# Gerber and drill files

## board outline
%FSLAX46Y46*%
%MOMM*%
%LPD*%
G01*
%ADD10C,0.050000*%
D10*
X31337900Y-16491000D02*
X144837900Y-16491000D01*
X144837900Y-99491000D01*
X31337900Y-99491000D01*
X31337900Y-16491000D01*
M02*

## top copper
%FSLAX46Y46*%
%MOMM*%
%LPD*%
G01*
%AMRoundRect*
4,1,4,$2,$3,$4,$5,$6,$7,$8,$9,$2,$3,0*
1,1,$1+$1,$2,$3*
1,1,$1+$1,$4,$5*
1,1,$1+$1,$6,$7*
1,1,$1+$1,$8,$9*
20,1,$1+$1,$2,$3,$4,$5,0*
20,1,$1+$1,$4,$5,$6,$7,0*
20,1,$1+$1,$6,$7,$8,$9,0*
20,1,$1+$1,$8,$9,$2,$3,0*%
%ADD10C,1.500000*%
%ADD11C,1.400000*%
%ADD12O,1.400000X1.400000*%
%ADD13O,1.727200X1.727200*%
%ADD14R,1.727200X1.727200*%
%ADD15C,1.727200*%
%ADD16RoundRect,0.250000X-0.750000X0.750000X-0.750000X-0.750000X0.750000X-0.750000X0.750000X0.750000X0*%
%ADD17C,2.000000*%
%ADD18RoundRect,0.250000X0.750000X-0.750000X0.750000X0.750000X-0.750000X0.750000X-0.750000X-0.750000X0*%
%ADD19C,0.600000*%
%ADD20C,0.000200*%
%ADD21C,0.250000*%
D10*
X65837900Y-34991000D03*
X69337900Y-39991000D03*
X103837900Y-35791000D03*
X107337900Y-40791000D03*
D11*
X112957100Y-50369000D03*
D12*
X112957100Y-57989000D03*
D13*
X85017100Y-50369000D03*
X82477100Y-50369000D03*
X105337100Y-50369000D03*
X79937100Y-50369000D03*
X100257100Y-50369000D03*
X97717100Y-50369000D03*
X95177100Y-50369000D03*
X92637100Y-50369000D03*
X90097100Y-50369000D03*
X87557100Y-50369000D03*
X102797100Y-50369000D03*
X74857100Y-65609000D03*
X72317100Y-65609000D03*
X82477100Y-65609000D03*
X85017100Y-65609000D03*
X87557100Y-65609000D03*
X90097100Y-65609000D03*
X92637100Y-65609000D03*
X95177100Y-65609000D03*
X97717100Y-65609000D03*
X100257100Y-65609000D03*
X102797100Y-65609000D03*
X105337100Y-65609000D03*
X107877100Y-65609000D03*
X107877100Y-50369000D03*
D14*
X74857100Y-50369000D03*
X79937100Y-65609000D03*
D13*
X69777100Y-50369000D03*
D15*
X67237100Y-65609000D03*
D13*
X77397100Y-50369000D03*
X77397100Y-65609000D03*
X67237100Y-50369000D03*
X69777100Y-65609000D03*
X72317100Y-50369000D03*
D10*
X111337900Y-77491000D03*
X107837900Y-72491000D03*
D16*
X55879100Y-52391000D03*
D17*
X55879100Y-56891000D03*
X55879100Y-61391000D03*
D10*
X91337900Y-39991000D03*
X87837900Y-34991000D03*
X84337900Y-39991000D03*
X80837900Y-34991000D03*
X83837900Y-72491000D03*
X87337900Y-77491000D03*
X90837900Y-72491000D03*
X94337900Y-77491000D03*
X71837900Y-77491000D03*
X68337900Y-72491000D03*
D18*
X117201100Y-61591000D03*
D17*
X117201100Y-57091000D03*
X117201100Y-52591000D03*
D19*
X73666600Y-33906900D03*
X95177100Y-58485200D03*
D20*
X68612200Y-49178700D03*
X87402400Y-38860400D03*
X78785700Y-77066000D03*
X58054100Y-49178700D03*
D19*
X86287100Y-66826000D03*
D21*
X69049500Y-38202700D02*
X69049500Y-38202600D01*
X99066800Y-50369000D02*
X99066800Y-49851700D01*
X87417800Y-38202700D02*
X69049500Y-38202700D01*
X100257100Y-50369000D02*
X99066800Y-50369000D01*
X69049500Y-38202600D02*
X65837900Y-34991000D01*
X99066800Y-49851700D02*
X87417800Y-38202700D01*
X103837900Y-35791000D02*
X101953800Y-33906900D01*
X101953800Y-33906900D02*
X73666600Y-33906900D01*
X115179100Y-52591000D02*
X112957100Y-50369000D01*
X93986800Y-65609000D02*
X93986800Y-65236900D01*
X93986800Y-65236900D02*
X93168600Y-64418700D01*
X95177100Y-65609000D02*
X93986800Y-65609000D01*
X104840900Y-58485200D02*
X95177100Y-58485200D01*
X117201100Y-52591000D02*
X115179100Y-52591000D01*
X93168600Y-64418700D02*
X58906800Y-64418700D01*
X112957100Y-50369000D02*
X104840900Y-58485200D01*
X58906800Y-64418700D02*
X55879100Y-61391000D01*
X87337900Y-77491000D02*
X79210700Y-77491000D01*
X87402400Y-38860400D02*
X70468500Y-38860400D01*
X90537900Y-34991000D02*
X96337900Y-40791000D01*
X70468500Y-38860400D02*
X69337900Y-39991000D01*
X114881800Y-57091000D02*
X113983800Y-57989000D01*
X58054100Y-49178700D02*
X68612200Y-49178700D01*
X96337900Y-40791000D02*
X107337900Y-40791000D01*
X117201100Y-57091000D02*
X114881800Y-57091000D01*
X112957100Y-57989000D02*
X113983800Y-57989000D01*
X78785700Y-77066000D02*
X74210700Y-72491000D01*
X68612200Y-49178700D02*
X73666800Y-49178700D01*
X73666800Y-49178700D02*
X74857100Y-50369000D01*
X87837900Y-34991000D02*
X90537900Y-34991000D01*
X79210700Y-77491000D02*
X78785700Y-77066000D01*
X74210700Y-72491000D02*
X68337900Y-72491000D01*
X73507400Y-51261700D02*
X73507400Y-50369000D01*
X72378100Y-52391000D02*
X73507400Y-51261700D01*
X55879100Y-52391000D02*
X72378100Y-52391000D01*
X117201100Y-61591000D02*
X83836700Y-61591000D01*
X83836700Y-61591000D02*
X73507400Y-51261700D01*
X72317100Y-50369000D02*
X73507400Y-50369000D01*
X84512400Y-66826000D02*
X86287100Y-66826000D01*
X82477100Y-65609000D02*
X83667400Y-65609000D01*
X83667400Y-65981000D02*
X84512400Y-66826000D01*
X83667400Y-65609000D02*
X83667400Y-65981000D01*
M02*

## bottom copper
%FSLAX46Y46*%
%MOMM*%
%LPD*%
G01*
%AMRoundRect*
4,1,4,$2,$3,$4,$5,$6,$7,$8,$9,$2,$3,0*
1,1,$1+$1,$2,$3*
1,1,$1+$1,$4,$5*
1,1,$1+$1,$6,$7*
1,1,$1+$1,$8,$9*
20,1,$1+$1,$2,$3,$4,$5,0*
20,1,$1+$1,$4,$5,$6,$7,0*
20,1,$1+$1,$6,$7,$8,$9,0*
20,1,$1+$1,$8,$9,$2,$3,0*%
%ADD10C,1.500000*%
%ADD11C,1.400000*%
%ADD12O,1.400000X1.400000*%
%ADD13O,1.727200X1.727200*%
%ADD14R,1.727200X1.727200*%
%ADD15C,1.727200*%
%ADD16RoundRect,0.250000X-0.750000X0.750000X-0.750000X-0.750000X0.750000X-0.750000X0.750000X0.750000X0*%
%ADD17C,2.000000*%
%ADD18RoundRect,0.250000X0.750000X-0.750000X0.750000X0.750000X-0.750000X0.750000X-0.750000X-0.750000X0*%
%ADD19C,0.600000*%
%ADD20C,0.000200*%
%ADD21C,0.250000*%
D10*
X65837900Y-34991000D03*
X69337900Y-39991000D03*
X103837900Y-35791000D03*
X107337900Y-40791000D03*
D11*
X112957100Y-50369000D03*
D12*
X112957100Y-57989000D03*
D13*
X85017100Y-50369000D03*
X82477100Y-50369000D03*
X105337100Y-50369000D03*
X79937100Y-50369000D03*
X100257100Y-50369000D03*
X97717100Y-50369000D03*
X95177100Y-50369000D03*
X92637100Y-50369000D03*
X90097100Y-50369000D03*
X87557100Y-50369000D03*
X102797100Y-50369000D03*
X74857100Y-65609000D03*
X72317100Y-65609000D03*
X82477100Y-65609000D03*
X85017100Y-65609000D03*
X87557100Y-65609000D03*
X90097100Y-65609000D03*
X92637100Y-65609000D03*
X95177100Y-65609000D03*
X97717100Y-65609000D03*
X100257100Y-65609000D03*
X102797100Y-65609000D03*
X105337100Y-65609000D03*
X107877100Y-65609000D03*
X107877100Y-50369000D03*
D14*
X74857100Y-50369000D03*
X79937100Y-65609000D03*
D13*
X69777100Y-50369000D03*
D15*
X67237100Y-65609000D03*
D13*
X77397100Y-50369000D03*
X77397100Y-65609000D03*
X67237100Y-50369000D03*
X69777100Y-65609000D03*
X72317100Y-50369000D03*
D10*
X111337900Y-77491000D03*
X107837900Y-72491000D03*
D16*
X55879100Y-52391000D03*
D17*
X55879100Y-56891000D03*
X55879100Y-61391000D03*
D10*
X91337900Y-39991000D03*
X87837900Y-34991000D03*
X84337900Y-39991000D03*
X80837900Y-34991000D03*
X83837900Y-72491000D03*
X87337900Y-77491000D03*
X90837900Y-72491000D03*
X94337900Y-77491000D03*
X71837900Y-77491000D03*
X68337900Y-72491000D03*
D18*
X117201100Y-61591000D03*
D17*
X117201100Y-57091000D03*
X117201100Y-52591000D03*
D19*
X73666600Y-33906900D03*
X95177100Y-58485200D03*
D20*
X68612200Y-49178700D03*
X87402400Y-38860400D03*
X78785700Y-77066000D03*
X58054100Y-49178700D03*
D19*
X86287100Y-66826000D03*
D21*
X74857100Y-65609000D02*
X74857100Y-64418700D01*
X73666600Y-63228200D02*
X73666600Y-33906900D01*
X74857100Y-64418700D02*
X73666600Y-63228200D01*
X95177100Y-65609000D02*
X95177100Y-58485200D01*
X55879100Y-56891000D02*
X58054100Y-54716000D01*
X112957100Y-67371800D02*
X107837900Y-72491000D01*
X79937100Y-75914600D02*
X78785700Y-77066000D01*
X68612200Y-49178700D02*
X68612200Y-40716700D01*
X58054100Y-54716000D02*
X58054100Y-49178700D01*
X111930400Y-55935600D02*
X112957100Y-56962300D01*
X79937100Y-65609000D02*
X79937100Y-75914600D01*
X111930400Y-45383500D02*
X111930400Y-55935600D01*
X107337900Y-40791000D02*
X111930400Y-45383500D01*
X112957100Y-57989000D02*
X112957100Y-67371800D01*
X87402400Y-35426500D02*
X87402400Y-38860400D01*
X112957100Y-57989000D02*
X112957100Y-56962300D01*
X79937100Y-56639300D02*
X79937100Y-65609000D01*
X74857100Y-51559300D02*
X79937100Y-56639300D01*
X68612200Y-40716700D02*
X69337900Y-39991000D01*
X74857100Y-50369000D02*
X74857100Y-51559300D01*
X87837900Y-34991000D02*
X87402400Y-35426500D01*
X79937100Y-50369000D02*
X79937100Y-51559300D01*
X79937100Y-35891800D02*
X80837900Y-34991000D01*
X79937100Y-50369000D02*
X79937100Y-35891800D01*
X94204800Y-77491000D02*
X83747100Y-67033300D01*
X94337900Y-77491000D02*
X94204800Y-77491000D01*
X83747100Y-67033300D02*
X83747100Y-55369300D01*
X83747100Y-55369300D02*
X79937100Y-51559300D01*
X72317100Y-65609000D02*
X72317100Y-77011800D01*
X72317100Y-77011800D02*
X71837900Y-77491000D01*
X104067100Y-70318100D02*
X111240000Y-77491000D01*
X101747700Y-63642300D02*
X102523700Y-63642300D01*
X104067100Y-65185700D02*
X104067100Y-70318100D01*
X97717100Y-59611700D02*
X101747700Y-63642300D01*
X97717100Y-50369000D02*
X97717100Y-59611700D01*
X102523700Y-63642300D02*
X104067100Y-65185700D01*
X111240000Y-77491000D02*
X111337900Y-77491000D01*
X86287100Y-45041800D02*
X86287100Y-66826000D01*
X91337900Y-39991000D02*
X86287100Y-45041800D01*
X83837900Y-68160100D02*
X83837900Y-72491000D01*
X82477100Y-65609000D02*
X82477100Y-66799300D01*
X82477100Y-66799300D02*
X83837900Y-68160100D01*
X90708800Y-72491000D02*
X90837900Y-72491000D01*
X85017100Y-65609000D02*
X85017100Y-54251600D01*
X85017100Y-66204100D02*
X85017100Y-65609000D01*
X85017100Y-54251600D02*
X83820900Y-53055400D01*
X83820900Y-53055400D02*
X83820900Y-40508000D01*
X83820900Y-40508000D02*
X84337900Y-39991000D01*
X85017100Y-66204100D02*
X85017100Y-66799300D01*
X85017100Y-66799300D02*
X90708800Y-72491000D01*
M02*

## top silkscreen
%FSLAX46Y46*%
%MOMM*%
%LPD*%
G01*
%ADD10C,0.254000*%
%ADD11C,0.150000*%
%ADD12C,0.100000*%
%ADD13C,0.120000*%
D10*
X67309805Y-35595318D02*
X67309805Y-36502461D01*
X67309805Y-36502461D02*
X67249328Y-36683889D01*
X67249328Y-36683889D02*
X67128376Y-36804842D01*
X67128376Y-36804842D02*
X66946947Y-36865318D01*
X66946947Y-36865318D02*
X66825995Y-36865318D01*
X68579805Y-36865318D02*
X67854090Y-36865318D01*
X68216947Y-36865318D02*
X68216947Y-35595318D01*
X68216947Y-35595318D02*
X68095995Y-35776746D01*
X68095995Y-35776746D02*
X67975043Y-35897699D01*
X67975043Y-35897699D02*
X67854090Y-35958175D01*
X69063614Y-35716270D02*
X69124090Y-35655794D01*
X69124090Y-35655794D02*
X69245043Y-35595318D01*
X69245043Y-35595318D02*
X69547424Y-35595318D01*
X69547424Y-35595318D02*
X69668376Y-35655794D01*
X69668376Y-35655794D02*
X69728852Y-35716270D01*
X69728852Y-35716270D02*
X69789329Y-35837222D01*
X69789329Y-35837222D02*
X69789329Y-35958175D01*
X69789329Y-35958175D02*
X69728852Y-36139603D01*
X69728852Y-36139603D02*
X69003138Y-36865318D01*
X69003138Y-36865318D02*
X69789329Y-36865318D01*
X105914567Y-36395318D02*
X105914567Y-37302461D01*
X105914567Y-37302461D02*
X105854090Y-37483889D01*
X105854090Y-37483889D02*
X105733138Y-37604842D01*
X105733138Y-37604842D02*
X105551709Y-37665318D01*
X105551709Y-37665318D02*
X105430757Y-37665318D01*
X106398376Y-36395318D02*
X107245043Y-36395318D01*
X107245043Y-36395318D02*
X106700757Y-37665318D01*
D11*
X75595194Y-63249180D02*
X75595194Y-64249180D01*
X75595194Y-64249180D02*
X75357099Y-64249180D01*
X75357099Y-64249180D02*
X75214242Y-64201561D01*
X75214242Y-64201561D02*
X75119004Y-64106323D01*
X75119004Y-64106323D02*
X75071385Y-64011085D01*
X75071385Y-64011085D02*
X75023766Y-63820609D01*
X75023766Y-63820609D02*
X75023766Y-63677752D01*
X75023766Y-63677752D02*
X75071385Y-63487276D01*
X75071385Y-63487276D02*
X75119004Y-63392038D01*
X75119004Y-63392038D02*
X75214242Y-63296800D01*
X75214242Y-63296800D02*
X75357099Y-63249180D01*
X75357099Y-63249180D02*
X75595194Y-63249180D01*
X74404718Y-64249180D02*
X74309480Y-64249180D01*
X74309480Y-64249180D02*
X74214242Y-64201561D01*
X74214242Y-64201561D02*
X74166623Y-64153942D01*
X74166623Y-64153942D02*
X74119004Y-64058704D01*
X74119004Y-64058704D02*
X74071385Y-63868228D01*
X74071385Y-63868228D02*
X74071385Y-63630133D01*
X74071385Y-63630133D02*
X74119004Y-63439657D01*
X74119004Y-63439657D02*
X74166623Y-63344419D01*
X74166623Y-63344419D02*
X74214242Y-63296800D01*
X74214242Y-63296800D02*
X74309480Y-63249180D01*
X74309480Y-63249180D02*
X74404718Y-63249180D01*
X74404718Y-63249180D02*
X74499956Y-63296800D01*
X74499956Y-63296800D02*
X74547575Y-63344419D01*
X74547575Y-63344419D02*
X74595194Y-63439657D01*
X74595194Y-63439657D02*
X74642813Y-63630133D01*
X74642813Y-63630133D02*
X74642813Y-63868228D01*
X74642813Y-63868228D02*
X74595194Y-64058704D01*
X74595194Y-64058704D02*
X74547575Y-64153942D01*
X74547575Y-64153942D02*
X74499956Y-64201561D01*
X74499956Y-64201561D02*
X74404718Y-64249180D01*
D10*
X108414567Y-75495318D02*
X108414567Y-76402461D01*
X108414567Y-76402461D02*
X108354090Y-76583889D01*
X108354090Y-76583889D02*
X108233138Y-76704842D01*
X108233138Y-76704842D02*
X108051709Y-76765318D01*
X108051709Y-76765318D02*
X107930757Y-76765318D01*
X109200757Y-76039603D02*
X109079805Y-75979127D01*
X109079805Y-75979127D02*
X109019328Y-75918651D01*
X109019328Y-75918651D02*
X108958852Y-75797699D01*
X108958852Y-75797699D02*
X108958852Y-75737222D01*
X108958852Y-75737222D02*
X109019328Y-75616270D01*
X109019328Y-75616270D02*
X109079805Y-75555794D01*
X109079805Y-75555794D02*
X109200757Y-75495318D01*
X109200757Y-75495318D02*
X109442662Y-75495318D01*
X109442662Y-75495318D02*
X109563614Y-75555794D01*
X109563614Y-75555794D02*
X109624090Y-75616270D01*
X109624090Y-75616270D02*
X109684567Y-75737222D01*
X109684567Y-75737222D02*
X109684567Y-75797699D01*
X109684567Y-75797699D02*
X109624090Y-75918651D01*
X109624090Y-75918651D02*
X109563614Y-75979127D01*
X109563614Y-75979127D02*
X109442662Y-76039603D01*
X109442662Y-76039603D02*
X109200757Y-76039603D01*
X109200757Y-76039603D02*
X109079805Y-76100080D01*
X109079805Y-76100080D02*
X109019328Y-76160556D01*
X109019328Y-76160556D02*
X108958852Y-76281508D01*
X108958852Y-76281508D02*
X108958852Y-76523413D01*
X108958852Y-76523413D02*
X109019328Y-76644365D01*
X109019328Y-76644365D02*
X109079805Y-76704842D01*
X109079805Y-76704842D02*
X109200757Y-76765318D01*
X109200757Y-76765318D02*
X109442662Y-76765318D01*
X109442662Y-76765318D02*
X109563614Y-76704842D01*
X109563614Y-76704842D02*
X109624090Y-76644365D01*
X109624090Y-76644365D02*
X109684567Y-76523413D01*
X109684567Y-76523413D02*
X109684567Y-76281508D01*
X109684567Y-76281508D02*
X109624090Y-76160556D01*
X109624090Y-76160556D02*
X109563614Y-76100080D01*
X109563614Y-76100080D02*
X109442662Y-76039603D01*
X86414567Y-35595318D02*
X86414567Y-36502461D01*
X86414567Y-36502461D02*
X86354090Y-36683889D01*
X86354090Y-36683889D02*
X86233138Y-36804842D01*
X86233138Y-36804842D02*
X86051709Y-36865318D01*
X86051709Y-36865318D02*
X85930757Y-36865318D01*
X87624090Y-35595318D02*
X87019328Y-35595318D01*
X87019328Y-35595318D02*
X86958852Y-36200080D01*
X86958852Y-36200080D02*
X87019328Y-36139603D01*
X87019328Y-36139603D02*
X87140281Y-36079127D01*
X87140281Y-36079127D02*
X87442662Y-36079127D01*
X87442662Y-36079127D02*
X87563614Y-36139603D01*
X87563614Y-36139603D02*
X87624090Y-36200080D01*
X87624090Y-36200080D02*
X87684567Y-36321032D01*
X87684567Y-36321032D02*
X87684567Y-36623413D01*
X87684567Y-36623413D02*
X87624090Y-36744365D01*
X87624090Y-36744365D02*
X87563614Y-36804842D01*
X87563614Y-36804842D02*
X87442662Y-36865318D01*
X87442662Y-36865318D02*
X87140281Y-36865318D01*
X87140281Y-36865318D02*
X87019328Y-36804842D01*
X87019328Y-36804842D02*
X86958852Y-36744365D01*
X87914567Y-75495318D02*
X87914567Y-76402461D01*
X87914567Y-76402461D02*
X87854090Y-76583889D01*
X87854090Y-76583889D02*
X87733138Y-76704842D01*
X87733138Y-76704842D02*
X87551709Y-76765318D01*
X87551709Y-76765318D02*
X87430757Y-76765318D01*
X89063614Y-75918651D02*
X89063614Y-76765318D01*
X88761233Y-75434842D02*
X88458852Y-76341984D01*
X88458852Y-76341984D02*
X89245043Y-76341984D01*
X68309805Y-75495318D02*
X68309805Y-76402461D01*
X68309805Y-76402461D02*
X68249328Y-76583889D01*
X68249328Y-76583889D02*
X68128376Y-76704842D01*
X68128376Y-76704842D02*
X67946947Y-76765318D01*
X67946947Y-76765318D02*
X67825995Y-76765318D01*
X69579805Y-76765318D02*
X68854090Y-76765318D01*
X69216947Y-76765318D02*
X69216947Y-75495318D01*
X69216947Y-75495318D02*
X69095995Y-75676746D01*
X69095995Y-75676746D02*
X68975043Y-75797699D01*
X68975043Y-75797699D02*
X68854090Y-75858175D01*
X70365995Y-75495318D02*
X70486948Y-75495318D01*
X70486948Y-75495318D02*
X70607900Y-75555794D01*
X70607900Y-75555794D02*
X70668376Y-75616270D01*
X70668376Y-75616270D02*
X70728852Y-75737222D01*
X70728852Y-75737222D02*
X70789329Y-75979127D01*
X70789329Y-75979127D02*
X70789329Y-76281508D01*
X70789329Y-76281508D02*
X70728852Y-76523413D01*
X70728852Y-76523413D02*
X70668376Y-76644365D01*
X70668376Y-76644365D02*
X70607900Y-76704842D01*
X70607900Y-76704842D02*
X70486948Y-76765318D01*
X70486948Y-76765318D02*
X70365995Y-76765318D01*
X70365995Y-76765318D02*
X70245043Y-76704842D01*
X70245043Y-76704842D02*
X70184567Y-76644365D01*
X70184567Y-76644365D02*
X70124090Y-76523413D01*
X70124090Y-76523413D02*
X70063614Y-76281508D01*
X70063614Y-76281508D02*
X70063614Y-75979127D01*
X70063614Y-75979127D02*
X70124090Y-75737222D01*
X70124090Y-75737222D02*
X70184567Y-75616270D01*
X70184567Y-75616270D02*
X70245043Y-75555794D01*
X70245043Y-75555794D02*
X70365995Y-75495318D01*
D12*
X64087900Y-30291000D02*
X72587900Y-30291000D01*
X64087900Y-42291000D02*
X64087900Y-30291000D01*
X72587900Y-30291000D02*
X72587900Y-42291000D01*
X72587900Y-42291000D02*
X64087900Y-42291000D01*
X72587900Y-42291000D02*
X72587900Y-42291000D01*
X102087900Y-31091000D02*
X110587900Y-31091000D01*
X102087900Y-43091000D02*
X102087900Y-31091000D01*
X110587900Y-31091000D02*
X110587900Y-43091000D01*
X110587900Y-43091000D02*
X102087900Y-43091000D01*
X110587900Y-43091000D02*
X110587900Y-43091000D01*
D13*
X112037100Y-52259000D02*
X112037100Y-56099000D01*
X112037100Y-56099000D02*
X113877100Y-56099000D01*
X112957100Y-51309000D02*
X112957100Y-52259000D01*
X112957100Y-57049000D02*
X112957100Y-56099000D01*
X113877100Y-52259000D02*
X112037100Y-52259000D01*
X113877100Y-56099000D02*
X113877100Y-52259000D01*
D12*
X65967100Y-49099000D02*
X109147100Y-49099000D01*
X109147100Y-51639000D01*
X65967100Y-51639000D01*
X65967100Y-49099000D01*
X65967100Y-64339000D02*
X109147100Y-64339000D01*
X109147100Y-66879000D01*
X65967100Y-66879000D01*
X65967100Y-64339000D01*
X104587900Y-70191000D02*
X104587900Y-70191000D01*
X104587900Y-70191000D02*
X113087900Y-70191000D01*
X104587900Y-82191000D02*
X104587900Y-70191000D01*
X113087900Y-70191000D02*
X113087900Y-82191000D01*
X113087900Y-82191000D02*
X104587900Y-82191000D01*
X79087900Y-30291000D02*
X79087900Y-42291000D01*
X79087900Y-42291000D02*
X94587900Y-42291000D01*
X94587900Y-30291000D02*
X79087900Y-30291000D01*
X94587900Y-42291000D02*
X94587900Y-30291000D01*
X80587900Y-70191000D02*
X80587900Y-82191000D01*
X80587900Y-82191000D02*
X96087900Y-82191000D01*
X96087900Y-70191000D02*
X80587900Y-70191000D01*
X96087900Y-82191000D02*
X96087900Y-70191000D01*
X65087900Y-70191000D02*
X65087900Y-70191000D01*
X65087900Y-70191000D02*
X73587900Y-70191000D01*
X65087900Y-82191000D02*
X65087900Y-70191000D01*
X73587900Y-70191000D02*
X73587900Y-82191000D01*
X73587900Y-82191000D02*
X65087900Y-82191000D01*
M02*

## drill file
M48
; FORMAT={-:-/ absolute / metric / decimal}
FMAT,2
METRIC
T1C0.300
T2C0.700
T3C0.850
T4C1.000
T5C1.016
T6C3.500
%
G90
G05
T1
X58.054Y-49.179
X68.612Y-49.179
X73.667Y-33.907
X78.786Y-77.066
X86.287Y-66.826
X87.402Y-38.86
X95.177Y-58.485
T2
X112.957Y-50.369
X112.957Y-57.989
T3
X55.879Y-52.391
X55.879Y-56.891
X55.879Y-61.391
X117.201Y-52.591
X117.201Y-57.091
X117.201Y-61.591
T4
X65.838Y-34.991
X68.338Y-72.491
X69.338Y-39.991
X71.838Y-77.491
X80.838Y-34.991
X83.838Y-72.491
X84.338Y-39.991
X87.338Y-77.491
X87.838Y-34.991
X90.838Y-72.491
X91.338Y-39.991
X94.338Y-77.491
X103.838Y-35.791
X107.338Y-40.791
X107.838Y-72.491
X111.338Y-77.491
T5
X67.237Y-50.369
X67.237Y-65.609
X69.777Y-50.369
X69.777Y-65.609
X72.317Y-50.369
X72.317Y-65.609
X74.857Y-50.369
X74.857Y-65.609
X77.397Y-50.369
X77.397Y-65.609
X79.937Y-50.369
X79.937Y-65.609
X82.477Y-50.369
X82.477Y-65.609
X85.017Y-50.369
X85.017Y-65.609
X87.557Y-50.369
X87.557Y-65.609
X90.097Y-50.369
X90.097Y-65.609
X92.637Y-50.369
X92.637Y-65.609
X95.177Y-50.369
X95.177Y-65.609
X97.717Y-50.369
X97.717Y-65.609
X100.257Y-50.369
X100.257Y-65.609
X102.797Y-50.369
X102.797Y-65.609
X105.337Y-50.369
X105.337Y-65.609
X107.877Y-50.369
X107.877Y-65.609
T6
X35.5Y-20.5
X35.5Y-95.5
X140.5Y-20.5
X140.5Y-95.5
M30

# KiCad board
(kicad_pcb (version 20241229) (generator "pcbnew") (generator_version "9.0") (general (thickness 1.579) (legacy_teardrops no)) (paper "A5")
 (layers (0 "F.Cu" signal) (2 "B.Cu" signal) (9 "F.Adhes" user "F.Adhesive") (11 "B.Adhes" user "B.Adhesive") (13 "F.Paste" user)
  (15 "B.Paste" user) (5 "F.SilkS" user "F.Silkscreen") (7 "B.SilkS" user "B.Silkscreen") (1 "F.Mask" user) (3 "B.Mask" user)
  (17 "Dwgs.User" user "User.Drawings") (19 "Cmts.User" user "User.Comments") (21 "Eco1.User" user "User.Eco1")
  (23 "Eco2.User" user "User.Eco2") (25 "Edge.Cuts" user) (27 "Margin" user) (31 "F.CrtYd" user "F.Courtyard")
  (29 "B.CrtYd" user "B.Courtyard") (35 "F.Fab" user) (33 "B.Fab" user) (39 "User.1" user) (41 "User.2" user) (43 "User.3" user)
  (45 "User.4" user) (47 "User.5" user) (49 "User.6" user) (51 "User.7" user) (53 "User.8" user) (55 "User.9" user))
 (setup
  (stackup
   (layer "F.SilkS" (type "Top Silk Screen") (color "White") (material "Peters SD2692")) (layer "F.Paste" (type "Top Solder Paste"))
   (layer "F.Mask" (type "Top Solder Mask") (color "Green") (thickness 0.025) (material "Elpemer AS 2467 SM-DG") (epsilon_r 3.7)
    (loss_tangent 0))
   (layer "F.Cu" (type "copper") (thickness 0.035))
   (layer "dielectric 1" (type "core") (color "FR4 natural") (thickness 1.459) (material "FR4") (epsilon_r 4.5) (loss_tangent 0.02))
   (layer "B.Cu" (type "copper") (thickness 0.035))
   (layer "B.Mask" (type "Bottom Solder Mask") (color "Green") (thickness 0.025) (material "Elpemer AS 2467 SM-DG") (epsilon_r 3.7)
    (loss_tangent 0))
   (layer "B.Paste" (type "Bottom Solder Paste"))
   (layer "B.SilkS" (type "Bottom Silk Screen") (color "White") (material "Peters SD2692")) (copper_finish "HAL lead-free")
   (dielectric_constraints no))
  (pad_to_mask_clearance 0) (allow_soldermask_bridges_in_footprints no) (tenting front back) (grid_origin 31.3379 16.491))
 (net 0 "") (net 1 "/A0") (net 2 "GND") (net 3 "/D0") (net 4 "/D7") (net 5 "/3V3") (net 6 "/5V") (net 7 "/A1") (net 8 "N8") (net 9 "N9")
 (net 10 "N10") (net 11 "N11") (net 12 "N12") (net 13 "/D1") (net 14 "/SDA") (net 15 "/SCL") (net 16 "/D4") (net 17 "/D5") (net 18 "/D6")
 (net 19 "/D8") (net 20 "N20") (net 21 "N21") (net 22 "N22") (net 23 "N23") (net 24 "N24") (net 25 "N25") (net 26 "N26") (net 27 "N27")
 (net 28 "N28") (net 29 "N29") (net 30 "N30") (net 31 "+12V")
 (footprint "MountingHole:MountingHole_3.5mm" (layer "F.Cu") (at 35.5 95.5)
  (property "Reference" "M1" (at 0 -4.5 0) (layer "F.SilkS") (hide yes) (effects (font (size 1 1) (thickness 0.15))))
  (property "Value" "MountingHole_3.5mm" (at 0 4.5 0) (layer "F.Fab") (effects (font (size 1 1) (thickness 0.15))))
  (pad "" np_thru_hole circle (at 0 0) (size 3.5 3.5) (drill 3.5) (layers "*.Cu" "*.Mask")))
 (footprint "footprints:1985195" (layer "F.Cu") (at 72.5879 39.991 180)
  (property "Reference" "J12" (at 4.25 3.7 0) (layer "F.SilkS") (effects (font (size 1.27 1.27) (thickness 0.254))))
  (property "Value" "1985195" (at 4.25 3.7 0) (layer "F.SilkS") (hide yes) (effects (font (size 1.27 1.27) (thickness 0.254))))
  (fp_line (start 8.5 9.7) (end 0 9.7) (stroke (width 0.1) (type solid)) (layer "F.SilkS"))
  (fp_line (start 8.5 -2.3) (end 8.5 9.7) (stroke (width 0.1) (type solid)) (layer "F.SilkS"))
  (fp_line (start 0 9.7) (end 0 -2.3) (stroke (width 0.1) (type solid)) (layer "F.SilkS"))
  (fp_line (start 0 -2.3) (end 8.5 -2.3) (stroke (width 0.1) (type solid)) (layer "F.SilkS"))
  (fp_line (start 0 -2.3) (end 0 -2.3) (stroke (width 0.1) (type solid)) (layer "F.SilkS"))
  (pad "1" thru_hole circle (at 6.75 5 180) (size 1.5 1.5) (drill 1) (layers "*.Cu" "*.Mask") (remove_unused_layers no) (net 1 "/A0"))
  (pad "2" thru_hole circle (at 3.25 0 180) (size 1.5 1.5) (drill 1) (layers "*.Cu" "*.Mask") (remove_unused_layers no) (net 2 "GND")))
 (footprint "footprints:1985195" (layer "F.Cu") (at 110.5879 40.791 180)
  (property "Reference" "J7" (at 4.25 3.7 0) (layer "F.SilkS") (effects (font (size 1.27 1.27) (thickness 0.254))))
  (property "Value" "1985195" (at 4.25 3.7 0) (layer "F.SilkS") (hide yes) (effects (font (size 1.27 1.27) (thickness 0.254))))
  (fp_line (start 8.5 9.7) (end 0 9.7) (stroke (width 0.1) (type solid)) (layer "F.SilkS"))
  (fp_line (start 8.5 -2.3) (end 8.5 9.7) (stroke (width 0.1) (type solid)) (layer "F.SilkS"))
  (fp_line (start 0 9.7) (end 0 -2.3) (stroke (width 0.1) (type solid)) (layer "F.SilkS"))
  (fp_line (start 0 -2.3) (end 8.5 -2.3) (stroke (width 0.1) (type solid)) (layer "F.SilkS"))
  (fp_line (start 0 -2.3) (end 0 -2.3) (stroke (width 0.1) (type solid)) (layer "F.SilkS"))
  (pad "1" thru_hole circle (at 6.75 5 180) (size 1.5 1.5) (drill 1) (layers "*.Cu" "*.Mask") (remove_unused_layers no) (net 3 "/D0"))
  (pad "2" thru_hole circle (at 3.25 0 180) (size 1.5 1.5) (drill 1) (layers "*.Cu" "*.Mask") (remove_unused_layers no) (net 2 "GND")))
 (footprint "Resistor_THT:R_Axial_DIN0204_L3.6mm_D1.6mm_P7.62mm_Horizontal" (layer "F.Cu") (at 112.9571 50.369 -90)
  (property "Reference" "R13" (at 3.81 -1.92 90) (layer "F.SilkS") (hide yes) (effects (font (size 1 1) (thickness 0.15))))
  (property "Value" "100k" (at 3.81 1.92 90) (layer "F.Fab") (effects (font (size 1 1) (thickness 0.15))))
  (fp_line (start 1.89 0.92) (end 5.73 0.92) (stroke (width 0.12) (type solid)) (layer "F.SilkS"))
  (fp_line (start 5.73 0.92) (end 5.73 -0.92) (stroke (width 0.12) (type solid)) (layer "F.SilkS"))
  (fp_line (start 0.94 0) (end 1.89 0) (stroke (width 0.12) (type solid)) (layer "F.SilkS"))
  (fp_line (start 6.68 0) (end 5.73 0) (stroke (width 0.12) (type solid)) (layer "F.SilkS"))
  (fp_line (start 1.89 -0.92) (end 1.89 0.92) (stroke (width 0.12) (type solid)) (layer "F.SilkS"))
  (fp_line (start 5.73 -0.92) (end 1.89 -0.92) (stroke (width 0.12) (type solid)) (layer "F.SilkS"))
  (pad "1" thru_hole circle (at 0 0 270) (size 1.4 1.4) (drill 0.7) (layers "*.Cu" "*.Mask") (remove_unused_layers no) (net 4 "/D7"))
  (pad "2" thru_hole oval (at 7.62 0 270) (size 1.4 1.4) (drill 0.7) (layers "*.Cu" "*.Mask") (remove_unused_layers no) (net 2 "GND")))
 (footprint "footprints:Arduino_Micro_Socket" (layer "F.Cu") (at 111.7971 48.989 180)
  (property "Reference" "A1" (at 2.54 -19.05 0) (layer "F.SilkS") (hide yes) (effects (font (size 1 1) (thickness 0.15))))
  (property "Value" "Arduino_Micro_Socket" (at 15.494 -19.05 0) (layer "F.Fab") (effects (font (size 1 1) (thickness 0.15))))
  (fp_rect (start 2.65 -2.65) (end 45.83 -0.11) (stroke (width 0.1) (type default)) (fill no) (layer "F.SilkS"))
  (fp_rect (start 2.65 -17.89) (end 45.83 -15.35) (stroke (width 0.1) (type default)) (fill no) (layer "F.SilkS"))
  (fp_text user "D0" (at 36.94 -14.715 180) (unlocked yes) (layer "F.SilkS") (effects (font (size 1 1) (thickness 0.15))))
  (pad "" thru_hole oval (at 26.78 -1.38 180) (size 1.7272 1.7272) (drill 1.016) (layers "*.Cu" "*.Mask") (remove_unused_layers no))
  (pad "" thru_hole oval (at 29.32 -1.38 180) (size 1.7272 1.7272) (drill 1.016) (layers "*.Cu" "*.Mask") (remove_unused_layers no))
  (pad "3V3" thru_hole oval (at 6.46 -1.38 180) (size 1.7272 1.7272) (drill 1.016) (layers "*.Cu" "*.Mask") (remove_unused_layers no)
   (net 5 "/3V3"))
  (pad "5V" thru_hole oval (at 31.86 -1.38 180) (size 1.7272 1.7272) (drill 1.016) (layers "*.Cu" "*.Mask") (remove_unused_layers no)
   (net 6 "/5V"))
  (pad "A0" thru_hole oval (at 11.54 -1.38 180) (size 1.7272 1.7272) (drill 1.016) (layers "*.Cu" "*.Mask") (remove_unused_layers no)
   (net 1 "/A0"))
  (pad "A1" thru_hole oval (at 14.08 -1.38 180) (size 1.7272 1.7272) (drill 1.016) (layers "*.Cu" "*.Mask") (remove_unused_layers no)
   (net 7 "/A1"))
  (pad "A2" thru_hole oval (at 16.62 -1.38 180) (size 1.7272 1.7272) (drill 1.016) (layers "*.Cu" "*.Mask") (remove_unused_layers no)
   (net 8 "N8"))
  (pad "A3" thru_hole oval (at 19.16 -1.38 180) (size 1.7272 1.7272) (drill 1.016) (layers "*.Cu" "*.Mask") (remove_unused_layers no)
   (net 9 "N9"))
  (pad "A4" thru_hole oval (at 21.7 -1.38 180) (size 1.7272 1.7272) (drill 1.016) (layers "*.Cu" "*.Mask") (remove_unused_layers no)
   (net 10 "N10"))
  (pad "A5" thru_hole oval (at 24.24 -1.38 180) (size 1.7272 1.7272) (drill 1.016) (layers "*.Cu" "*.Mask") (remove_unused_layers no)
   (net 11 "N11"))
  (pad "AREF" thru_hole oval (at 9 -1.38 180) (size 1.7272 1.7272) (drill 1.016) (layers "*.Cu" "*.Mask") (remove_unused_layers no)
   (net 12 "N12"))
  (pad "D0" thru_hole oval (at 36.94 -16.62 180) (size 1.7272 1.7272) (drill 1.016) (layers "*.Cu" "*.Mask") (remove_unused_layers no)
   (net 3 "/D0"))
  (pad "D1" thru_hole oval (at 39.48 -16.62 180) (size 1.7272 1.7272) (drill 1.016) (layers "*.Cu" "*.Mask") (remove_unused_layers no)
   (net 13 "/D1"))
  (pad "D2" thru_hole oval (at 29.32 -16.62 180) (size 1.7272 1.7272) (drill 1.016) (layers "*.Cu" "*.Mask") (remove_unused_layers no)
   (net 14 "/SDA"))
  (pad "D3" thru_hole oval (at 26.78 -16.62 180) (size 1.7272 1.7272) (drill 1.016) (layers "*.Cu" "*.Mask") (remove_unused_layers no)
   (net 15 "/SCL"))
  (pad "D4" thru_hole oval (at 24.24 -16.62 180) (size 1.7272 1.7272) (drill 1.016) (layers "*.Cu" "*.Mask") (remove_unused_layers no)
   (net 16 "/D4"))
  (pad "D5" thru_hole oval (at 21.7 -16.62 180) (size 1.7272 1.7272) (drill 1.016) (layers "*.Cu" "*.Mask") (remove_unused_layers no)
   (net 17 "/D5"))
  (pad "D6" thru_hole oval (at 19.16 -16.62 180) (size 1.7272 1.7272) (drill 1.016) (layers "*.Cu" "*.Mask") (remove_unused_layers no)
   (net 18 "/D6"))
  (pad "D7" thru_hole oval (at 16.62 -16.62 180) (size 1.7272 1.7272) (drill 1.016) (layers "*.Cu" "*.Mask") (remove_unused_layers no)
   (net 4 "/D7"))
  (pad "D8" thru_hole oval (at 14.08 -16.62 180) (size 1.7272 1.7272) (drill 1.016) (layers "*.Cu" "*.Mask") (remove_unused_layers no)
   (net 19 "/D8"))
  (pad "D9" thru_hole oval (at 11.54 -16.62 180) (size 1.7272 1.7272) (drill 1.016) (layers "*.Cu" "*.Mask") (remove_unused_layers no)
   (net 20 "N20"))
  (pad "D10" thru_hole oval (at 9 -16.62 180) (size 1.7272 1.7272) (drill 1.016) (layers "*.Cu" "*.Mask") (remove_unused_layers no)
   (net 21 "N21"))
  (pad "D11" thru_hole oval (at 6.46 -16.62 180) (size 1.7272 1.7272) (drill 1.016) (layers "*.Cu" "*.Mask") (remove_unused_layers no)
   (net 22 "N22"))
  (pad "D12" thru_hole oval (at 3.92 -16.62 180) (size 1.7272 1.7272) (drill 1.016) (layers "*.Cu" "*.Mask") (remove_unused_layers no)
   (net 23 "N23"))
  (pad "D13" thru_hole oval (at 3.92 -1.38 180) (size 1.7272 1.7272) (drill 1.016) (layers "*.Cu" "*.Mask") (remove_unused_layers no)
   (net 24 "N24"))
  (pad "GND1" thru_hole rect (at 36.94 -1.38 180) (size 1.7272 1.7272) (drill 1.016) (layers "*.Cu" "*.Mask") (remove_unused_layers no)
   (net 2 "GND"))
  (pad "GND2" thru_hole rect (at 31.86 -16.62 180) (size 1.7272 1.7272) (drill 1.016) (layers "*.Cu" "*.Mask") (remove_unused_layers no)
   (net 2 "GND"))
  (pad "MISO" thru_hole oval (at 42.02 -1.38 180) (size 1.7272 1.7272) (drill 1.016) (layers "*.Cu" "*.Mask") (remove_unused_layers no)
   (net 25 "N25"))
  (pad "MOSI" thru_hole circle (at 44.56 -16.62 180) (size 1.7272 1.7272) (drill 1.016) (layers "*.Cu" "*.Mask") (remove_unused_layers no)
   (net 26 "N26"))
  (pad "RST1" thru_hole oval (at 34.4 -1.38 180) (size 1.7272 1.7272) (drill 1.016) (layers "*.Cu" "*.Mask") (remove_unused_layers no)
   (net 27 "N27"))
  (pad "RST2" thru_hole oval (at 34.4 -16.62 180) (size 1.7272 1.7272) (drill 1.016) (layers "*.Cu" "*.Mask") (remove_unused_layers no)
   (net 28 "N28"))
  (pad "SCK" thru_hole oval (at 44.56 -1.38 180) (size 1.7272 1.7272) (drill 1.016) (layers "*.Cu" "*.Mask") (remove_unused_layers no)
   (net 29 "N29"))
  (pad "SS" thru_hole oval (at 42.02 -16.62 180) (size 1.7272 1.7272) (drill 1.016) (layers "*.Cu" "*.Mask") (remove_unused_layers no)
   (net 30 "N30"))
  (pad "VIN" thru_hole oval (at 39.48 -1.38 180) (size 1.7272 1.7272) (drill 1.016) (layers "*.Cu" "*.Mask") (remove_unused_layers no)
   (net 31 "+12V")))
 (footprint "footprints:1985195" (layer "F.Cu") (at 104.5879 72.491)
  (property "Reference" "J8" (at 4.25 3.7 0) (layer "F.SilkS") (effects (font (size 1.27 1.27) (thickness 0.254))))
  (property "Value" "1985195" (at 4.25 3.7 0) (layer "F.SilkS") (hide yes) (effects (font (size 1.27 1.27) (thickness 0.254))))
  (fp_line (start 0 -2.3) (end 0 -2.3) (stroke (width 0.1) (type solid)) (layer "F.SilkS"))
  (fp_line (start 0 -2.3) (end 8.5 -2.3) (stroke (width 0.1) (type solid)) (layer "F.SilkS"))
  (fp_line (start 0 9.7) (end 0 -2.3) (stroke (width 0.1) (type solid)) (layer "F.SilkS"))
  (fp_line (start 8.5 -2.3) (end 8.5 9.7) (stroke (width 0.1) (type solid)) (layer "F.SilkS"))
  (fp_line (start 8.5 9.7) (end 0 9.7) (stroke (width 0.1) (type solid)) (layer "F.SilkS"))
  (pad "1" thru_hole circle (at 6.75 5) (size 1.5 1.5) (drill 1) (layers "*.Cu" "*.Mask") (remove_unused_layers no) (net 7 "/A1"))
  (pad "2" thru_hole circle (at 3.25 0) (size 1.5 1.5) (drill 1) (layers "*.Cu" "*.Mask") (remove_unused_layers no) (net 2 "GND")))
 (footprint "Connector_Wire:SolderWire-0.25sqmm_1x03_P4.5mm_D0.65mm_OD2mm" (layer "F.Cu") (at 55.8791 52.391 -90)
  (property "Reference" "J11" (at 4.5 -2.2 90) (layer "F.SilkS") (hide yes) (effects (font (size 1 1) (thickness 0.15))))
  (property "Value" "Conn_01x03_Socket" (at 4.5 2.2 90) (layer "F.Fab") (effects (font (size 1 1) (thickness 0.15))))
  (pad "1" thru_hole roundrect (at 0 0 270) (size 2 2) (drill 0.85) (layers "*.Cu" "*.Mask") (remove_unused_layers no)
   (roundrect_rratio 0.125) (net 31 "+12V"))
  (pad "2" thru_hole circle (at 4.5 0 270) (size 2 2) (drill 0.85) (layers "*.Cu" "*.Mask") (remove_unused_layers no) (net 2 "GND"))
  (pad "3" thru_hole circle (at 9 0 270) (size 2 2) (drill 0.85) (layers "*.Cu" "*.Mask") (remove_unused_layers no) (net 4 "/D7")))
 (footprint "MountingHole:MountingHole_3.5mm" (layer "F.Cu") (at 35.5 20.5)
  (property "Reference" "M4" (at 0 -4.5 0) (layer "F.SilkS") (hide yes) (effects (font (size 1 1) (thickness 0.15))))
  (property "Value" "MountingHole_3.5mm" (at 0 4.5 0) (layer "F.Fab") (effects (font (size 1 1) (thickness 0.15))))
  (pad "" np_thru_hole circle (at 0 0) (size 3.5 3.5) (drill 3.5) (layers "*.Cu" "*.Mask")))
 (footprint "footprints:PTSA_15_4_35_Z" (layer "F.Cu") (at 91.3379 39.991 180)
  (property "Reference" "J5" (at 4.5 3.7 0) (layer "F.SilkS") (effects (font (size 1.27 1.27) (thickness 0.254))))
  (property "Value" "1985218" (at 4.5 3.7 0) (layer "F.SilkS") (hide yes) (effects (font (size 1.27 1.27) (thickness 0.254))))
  (fp_line (start 12.25 9.7) (end 12.25 -2.3) (stroke (width 0.1) (type solid)) (layer "F.SilkS"))
  (fp_line (start 12.25 -2.3) (end -3.25 -2.3) (stroke (width 0.1) (type solid)) (layer "F.SilkS"))
  (fp_line (start -3.25 9.7) (end 12.25 9.7) (stroke (width 0.1) (type solid)) (layer "F.SilkS"))
  (fp_line (start -3.25 -2.3) (end -3.25 9.7) (stroke (width 0.1) (type solid)) (layer "F.SilkS"))
  (pad "1" thru_hole circle (at 0 0 180) (size 1.5 1.5) (drill 1) (layers "*.Cu" "*.Mask") (remove_unused_layers no) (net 14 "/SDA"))
  (pad "2" thru_hole circle (at 3.5 5 180) (size 1.5 1.5) (drill 1) (layers "*.Cu" "*.Mask") (remove_unused_layers no) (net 2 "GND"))
  (pad "3" thru_hole circle (at 7 0 180) (size 1.5 1.5) (drill 1) (layers "*.Cu" "*.Mask") (remove_unused_layers no) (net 15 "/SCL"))
  (pad "4" thru_hole circle (at 10.5 5 180) (size 1.5 1.5) (drill 1) (layers "*.Cu" "*.Mask") (remove_unused_layers no) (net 6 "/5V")))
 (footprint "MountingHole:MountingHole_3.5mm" (layer "F.Cu") (at 140.5 95.5)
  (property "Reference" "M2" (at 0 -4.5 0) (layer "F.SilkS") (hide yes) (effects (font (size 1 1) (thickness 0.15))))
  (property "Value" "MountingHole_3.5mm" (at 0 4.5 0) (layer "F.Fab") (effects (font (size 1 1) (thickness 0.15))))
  (pad "" np_thru_hole circle (at 0 0) (size 3.5 3.5) (drill 3.5) (layers "*.Cu" "*.Mask")))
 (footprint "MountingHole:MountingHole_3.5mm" (layer "F.Cu") (at 140.5 20.5)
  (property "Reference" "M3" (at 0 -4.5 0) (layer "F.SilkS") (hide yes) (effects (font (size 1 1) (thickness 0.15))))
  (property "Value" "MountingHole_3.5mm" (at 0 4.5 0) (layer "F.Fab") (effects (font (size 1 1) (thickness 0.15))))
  (pad "" np_thru_hole circle (at 0 0) (size 3.5 3.5) (drill 3.5) (layers "*.Cu" "*.Mask")))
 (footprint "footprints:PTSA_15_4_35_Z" (layer "F.Cu") (at 83.8379 72.491)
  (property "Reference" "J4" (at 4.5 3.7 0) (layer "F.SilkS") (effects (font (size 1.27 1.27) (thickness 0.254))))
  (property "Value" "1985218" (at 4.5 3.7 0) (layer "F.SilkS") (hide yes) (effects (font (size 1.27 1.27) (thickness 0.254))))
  (fp_line (start -3.25 -2.3) (end -3.25 9.7) (stroke (width 0.1) (type solid)) (layer "F.SilkS"))
  (fp_line (start -3.25 9.7) (end 12.25 9.7) (stroke (width 0.1) (type solid)) (layer "F.SilkS"))
  (fp_line (start 12.25 -2.3) (end -3.25 -2.3) (stroke (width 0.1) (type solid)) (layer "F.SilkS"))
  (fp_line (start 12.25 9.7) (end 12.25 -2.3) (stroke (width 0.1) (type solid)) (layer "F.SilkS"))
  (pad "1" thru_hole circle (at 0 0) (size 1.5 1.5) (drill 1) (layers "*.Cu" "*.Mask") (remove_unused_layers no) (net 14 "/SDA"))
  (pad "2" thru_hole circle (at 3.5 5) (size 1.5 1.5) (drill 1) (layers "*.Cu" "*.Mask") (remove_unused_layers no) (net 2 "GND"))
  (pad "3" thru_hole circle (at 7 0) (size 1.5 1.5) (drill 1) (layers "*.Cu" "*.Mask") (remove_unused_layers no) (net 15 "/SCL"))
  (pad "4" thru_hole circle (at 10.5 5) (size 1.5 1.5) (drill 1) (layers "*.Cu" "*.Mask") (remove_unused_layers no) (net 6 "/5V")))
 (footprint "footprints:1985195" (layer "F.Cu") (at 65.0879 72.491)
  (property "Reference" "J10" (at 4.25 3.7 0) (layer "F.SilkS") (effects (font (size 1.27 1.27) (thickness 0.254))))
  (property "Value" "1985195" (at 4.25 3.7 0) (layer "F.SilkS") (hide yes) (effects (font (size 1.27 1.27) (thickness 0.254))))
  (fp_line (start 0 -2.3) (end 0 -2.3) (stroke (width 0.1) (type solid)) (layer "F.SilkS"))
  (fp_line (start 0 -2.3) (end 8.5 -2.3) (stroke (width 0.1) (type solid)) (layer "F.SilkS"))
  (fp_line (start 0 9.7) (end 0 -2.3) (stroke (width 0.1) (type solid)) (layer "F.SilkS"))
  (fp_line (start 8.5 -2.3) (end 8.5 9.7) (stroke (width 0.1) (type solid)) (layer "F.SilkS"))
  (fp_line (start 8.5 9.7) (end 0 9.7) (stroke (width 0.1) (type solid)) (layer "F.SilkS"))
  (pad "1" thru_hole circle (at 6.75 5) (size 1.5 1.5) (drill 1) (layers "*.Cu" "*.Mask") (remove_unused_layers no) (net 13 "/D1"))
  (pad "2" thru_hole circle (at 3.25 0) (size 1.5 1.5) (drill 1) (layers "*.Cu" "*.Mask") (remove_unused_layers no) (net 2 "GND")))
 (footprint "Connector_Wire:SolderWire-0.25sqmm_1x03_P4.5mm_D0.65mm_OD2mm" (layer "F.Cu") (at 117.2011 61.591 90)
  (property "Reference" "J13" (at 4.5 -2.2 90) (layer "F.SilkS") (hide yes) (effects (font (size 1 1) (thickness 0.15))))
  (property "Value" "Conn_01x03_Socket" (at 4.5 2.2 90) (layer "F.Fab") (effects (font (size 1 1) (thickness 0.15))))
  (pad "1" thru_hole roundrect (at 0 0 90) (size 2 2) (drill 0.85) (layers "*.Cu" "*.Mask") (remove_unused_layers no)
   (roundrect_rratio 0.125) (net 31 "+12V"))
  (pad "2" thru_hole circle (at 4.5 0 90) (size 2 2) (drill 0.85) (layers "*.Cu" "*.Mask") (remove_unused_layers no) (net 2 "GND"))
  (pad "3" thru_hole circle (at 9 0 90) (size 2 2) (drill 0.85) (layers "*.Cu" "*.Mask") (remove_unused_layers no) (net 4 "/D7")))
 (gr_rect (start 31.3379 16.491) (end 144.8379 99.491) (stroke (width 0.05) (type solid)) (fill no) (layer "Edge.Cuts"))
 (segment (start 69.0495 38.2027) (end 69.0495 38.2026) (width 0.25) (layer "F.Cu") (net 1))
 (segment (start 99.0668 50.369) (end 99.0668 49.8517) (width 0.25) (layer "F.Cu") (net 1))
 (segment (start 87.4178 38.2027) (end 69.0495 38.2027) (width 0.25) (layer "F.Cu") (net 1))
 (segment (start 100.2571 50.369) (end 99.0668 50.369) (width 0.25) (layer "F.Cu") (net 1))
 (segment (start 69.0495 38.2026) (end 65.8379 34.991) (width 0.25) (layer "F.Cu") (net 1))
 (segment (start 99.0668 49.8517) (end 87.4178 38.2027) (width 0.25) (layer "F.Cu") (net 1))
 (segment (start 103.8379 35.791) (end 101.9538 33.9069) (width 0.25) (layer "F.Cu") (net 3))
 (segment (start 101.9538 33.9069) (end 73.6666 33.9069) (width 0.25) (layer "F.Cu") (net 3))
 (via (at 73.6666 33.9069) (size 0.6) (drill 0.3) (layers "F.Cu" "B.Cu") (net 3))
 (segment (start 74.8571 65.609) (end 74.8571 64.4187) (width 0.25) (layer "B.Cu") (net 3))
 (segment (start 73.6666 63.2282) (end 73.6666 33.9069) (width 0.25) (layer "B.Cu") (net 3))
 (segment (start 74.8571 64.4187) (end 73.6666 63.2282) (width 0.25) (layer "B.Cu") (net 3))
 (segment (start 115.1791 52.591) (end 112.9571 50.369) (width 0.25) (layer "F.Cu") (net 4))
 (segment (start 93.9868 65.609) (end 93.9868 65.2369) (width 0.25) (layer "F.Cu") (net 4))
 (segment (start 93.9868 65.2369) (end 93.1686 64.4187) (width 0.25) (layer "F.Cu") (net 4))
 (segment (start 95.1771 65.609) (end 93.9868 65.609) (width 0.25) (layer "F.Cu") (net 4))
 (segment (start 104.8409 58.4852) (end 95.1771 58.4852) (width 0.25) (layer "F.Cu") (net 4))
 (segment (start 117.2011 52.591) (end 115.1791 52.591) (width 0.25) (layer "F.Cu") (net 4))
 (segment (start 93.1686 64.4187) (end 58.9068 64.4187) (width 0.25) (layer "F.Cu") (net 4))
 (segment (start 112.9571 50.369) (end 104.8409 58.4852) (width 0.25) (layer "F.Cu") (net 4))
 (segment (start 58.9068 64.4187) (end 55.8791 61.391) (width 0.25) (layer "F.Cu") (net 4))
 (via (at 95.1771 58.4852) (size 0.6) (drill 0.3) (layers "F.Cu" "B.Cu") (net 4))
 (segment (start 95.1771 65.609) (end 95.1771 58.4852) (width 0.25) (layer "B.Cu") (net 4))
 (segment (start 87.3379 77.491) (end 79.2107 77.491) (width 0.25) (layer "F.Cu") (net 2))
 (segment (start 87.4024 38.8604) (end 70.4685 38.8604) (width 0.25) (layer "F.Cu") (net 2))
 (segment (start 90.5379 34.991) (end 96.3379 40.791) (width 0.25) (layer "F.Cu") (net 2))
 (segment (start 70.4685 38.8604) (end 69.3379 39.991) (width 0.25) (layer "F.Cu") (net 2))
 (segment (start 114.8818 57.091) (end 113.9838 57.989) (width 0.25) (layer "F.Cu") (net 2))
 (segment (start 58.0541 49.1787) (end 68.6122 49.1787) (width 0.25) (layer "F.Cu") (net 2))
 (segment (start 96.3379 40.791) (end 107.3379 40.791) (width 0.25) (layer "F.Cu") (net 2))
 (segment (start 117.2011 57.091) (end 114.8818 57.091) (width 0.25) (layer "F.Cu") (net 2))
 (segment (start 112.9571 57.989) (end 113.9838 57.989) (width 0.25) (layer "F.Cu") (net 2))
 (segment (start 78.7857 77.066) (end 74.2107 72.491) (width 0.25) (layer "F.Cu") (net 2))
 (segment (start 68.6122 49.1787) (end 73.6668 49.1787) (width 0.25) (layer "F.Cu") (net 2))
 (segment (start 73.6668 49.1787) (end 74.8571 50.369) (width 0.25) (layer "F.Cu") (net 2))
 (segment (start 87.8379 34.991) (end 90.5379 34.991) (width 0.25) (layer "F.Cu") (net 2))
 (segment (start 79.2107 77.491) (end 78.7857 77.066) (width 0.25) (layer "F.Cu") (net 2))
 (segment (start 74.2107 72.491) (end 68.3379 72.491) (width 0.25) (layer "F.Cu") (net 2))
 (via (at 68.6122 49.1787) (size 0.0002) (drill 0.3) (layers "F.Cu" "B.Cu") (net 2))
 (via (at 87.4024 38.8604) (size 0.0002) (drill 0.3) (layers "F.Cu" "B.Cu") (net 2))
 (via (at 78.7857 77.066) (size 0.0002) (drill 0.3) (layers "F.Cu" "B.Cu") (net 2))
 (via (at 58.0541 49.1787) (size 0.0002) (drill 0.3) (layers "F.Cu" "B.Cu") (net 2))
 (segment (start 55.8791 56.891) (end 58.0541 54.716) (width 0.25) (layer "B.Cu") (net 2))
 (segment (start 112.9571 67.3718) (end 107.8379 72.491) (width 0.25) (layer "B.Cu") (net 2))
 (segment (start 79.9371 75.9146) (end 78.7857 77.066) (width 0.25) (layer "B.Cu") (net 2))
 (segment (start 68.6122 49.1787) (end 68.6122 40.7167) (width 0.25) (layer "B.Cu") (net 2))
 (segment (start 58.0541 54.716) (end 58.0541 49.1787) (width 0.25) (layer "B.Cu") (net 2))
 (segment (start 111.9304 55.9356) (end 112.9571 56.9623) (width 0.25) (layer "B.Cu") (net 2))
 (segment (start 79.9371 65.609) (end 79.9371 75.9146) (width 0.25) (layer "B.Cu") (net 2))
 (segment (start 111.9304 45.3835) (end 111.9304 55.9356) (width 0.25) (layer "B.Cu") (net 2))
 (segment (start 107.3379 40.791) (end 111.9304 45.3835) (width 0.25) (layer "B.Cu") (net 2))
 (segment (start 112.9571 57.989) (end 112.9571 67.3718) (width 0.25) (layer "B.Cu") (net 2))
 (segment (start 87.4024 35.4265) (end 87.4024 38.8604) (width 0.25) (layer "B.Cu") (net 2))
 (segment (start 112.9571 57.989) (end 112.9571 56.9623) (width 0.25) (layer "B.Cu") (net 2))
 (segment (start 79.9371 56.6393) (end 79.9371 65.609) (width 0.25) (layer "B.Cu") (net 2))
 (segment (start 74.8571 51.5593) (end 79.9371 56.6393) (width 0.25) (layer "B.Cu") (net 2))
 (segment (start 68.6122 40.7167) (end 69.3379 39.991) (width 0.25) (layer "B.Cu") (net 2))
 (segment (start 74.8571 50.369) (end 74.8571 51.5593) (width 0.25) (layer "B.Cu") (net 2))
 (segment (start 87.8379 34.991) (end 87.4024 35.4265) (width 0.25) (layer "B.Cu") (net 2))
 (segment (start 73.5074 51.2617) (end 73.5074 50.369) (width 0.25) (layer "F.Cu") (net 31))
 (segment (start 72.3781 52.391) (end 73.5074 51.2617) (width 0.25) (layer "F.Cu") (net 31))
 (segment (start 55.8791 52.391) (end 72.3781 52.391) (width 0.25) (layer "F.Cu") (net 31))
 (segment (start 117.2011 61.591) (end 83.8367 61.591) (width 0.25) (layer "F.Cu") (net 31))
 (segment (start 83.8367 61.591) (end 73.5074 51.2617) (width 0.25) (layer "F.Cu") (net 31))
 (segment (start 72.3171 50.369) (end 73.5074 50.369) (width 0.25) (layer "F.Cu") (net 31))
 (segment (start 79.9371 50.369) (end 79.9371 51.5593) (width 0.25) (layer "B.Cu") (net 6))
 (segment (start 79.9371 35.8918) (end 80.8379 34.991) (width 0.25) (layer "B.Cu") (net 6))
 (segment (start 79.9371 50.369) (end 79.9371 35.8918) (width 0.25) (layer "B.Cu") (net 6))
 (segment (start 94.2048 77.491) (end 83.7471 67.0333) (width 0.25) (layer "B.Cu") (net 6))
 (segment (start 94.3379 77.491) (end 94.2048 77.491) (width 0.25) (layer "B.Cu") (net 6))
 (segment (start 83.7471 67.0333) (end 83.7471 55.3693) (width 0.25) (layer "B.Cu") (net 6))
 (segment (start 83.7471 55.3693) (end 79.9371 51.5593) (width 0.25) (layer "B.Cu") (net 6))
 (segment (start 72.3171 65.609) (end 72.3171 77.0118) (width 0.25) (layer "B.Cu") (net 13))
 (segment (start 72.3171 77.0118) (end 71.8379 77.491) (width 0.25) (layer "B.Cu") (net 13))
 (segment (start 104.0671 70.3181) (end 111.24 77.491) (width 0.25) (layer "B.Cu") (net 7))
 (segment (start 101.7477 63.6423) (end 102.5237 63.6423) (width 0.25) (layer "B.Cu") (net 7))
 (segment (start 104.0671 65.1857) (end 104.0671 70.3181) (width 0.25) (layer "B.Cu") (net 7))
 (segment (start 97.7171 59.6117) (end 101.7477 63.6423) (width 0.25) (layer "B.Cu") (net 7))
 (segment (start 97.7171 50.369) (end 97.7171 59.6117) (width 0.25) (layer "B.Cu") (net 7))
 (segment (start 102.5237 63.6423) (end 104.0671 65.1857) (width 0.25) (layer "B.Cu") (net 7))
 (segment (start 111.24 77.491) (end 111.3379 77.491) (width 0.25) (layer "B.Cu") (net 7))
 (segment (start 84.5124 66.826) (end 86.2871 66.826) (width 0.25) (layer "F.Cu") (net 14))
 (segment (start 82.4771 65.609) (end 83.6674 65.609) (width 0.25) (layer "F.Cu") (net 14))
 (segment (start 83.6674 65.981) (end 84.5124 66.826) (width 0.25) (layer "F.Cu") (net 14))
 (segment (start 83.6674 65.609) (end 83.6674 65.981) (width 0.25) (layer "F.Cu") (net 14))
 (via (at 86.2871 66.826) (size 0.6) (drill 0.3) (layers "F.Cu" "B.Cu") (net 14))
 (segment (start 86.2871 45.0418) (end 86.2871 66.826) (width 0.25) (layer "B.Cu") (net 14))
 (segment (start 91.3379 39.991) (end 86.2871 45.0418) (width 0.25) (layer "B.Cu") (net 14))
 (segment (start 83.8379 68.1601) (end 83.8379 72.491) (width 0.25) (layer "B.Cu") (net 14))
 (segment (start 82.4771 65.609) (end 82.4771 66.7993) (width 0.25) (layer "B.Cu") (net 14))
 (segment (start 82.4771 66.7993) (end 83.8379 68.1601) (width 0.25) (layer "B.Cu") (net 14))
 (segment (start 90.7088 72.491) (end 90.8379 72.491) (width 0.25) (layer "B.Cu") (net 15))
 (segment (start 85.0171 65.609) (end 85.0171 54.2516) (width 0.25) (layer "B.Cu") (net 15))
 (segment (start 85.0171 66.2041) (end 85.0171 65.609) (width 0.25) (layer "B.Cu") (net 15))
 (segment (start 85.0171 54.2516) (end 83.8209 53.0554) (width 0.25) (layer "B.Cu") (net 15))
 (segment (start 83.8209 53.0554) (end 83.8209 40.508) (width 0.25) (layer "B.Cu") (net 15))
 (segment (start 83.8209 40.508) (end 84.3379 39.991) (width 0.25) (layer "B.Cu") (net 15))
 (segment (start 85.0171 66.2041) (end 85.0171 66.7993) (width 0.25) (layer "B.Cu") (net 15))
 (segment (start 85.0171 66.7993) (end 90.7088 72.491) (width 0.25) (layer "B.Cu") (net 15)))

